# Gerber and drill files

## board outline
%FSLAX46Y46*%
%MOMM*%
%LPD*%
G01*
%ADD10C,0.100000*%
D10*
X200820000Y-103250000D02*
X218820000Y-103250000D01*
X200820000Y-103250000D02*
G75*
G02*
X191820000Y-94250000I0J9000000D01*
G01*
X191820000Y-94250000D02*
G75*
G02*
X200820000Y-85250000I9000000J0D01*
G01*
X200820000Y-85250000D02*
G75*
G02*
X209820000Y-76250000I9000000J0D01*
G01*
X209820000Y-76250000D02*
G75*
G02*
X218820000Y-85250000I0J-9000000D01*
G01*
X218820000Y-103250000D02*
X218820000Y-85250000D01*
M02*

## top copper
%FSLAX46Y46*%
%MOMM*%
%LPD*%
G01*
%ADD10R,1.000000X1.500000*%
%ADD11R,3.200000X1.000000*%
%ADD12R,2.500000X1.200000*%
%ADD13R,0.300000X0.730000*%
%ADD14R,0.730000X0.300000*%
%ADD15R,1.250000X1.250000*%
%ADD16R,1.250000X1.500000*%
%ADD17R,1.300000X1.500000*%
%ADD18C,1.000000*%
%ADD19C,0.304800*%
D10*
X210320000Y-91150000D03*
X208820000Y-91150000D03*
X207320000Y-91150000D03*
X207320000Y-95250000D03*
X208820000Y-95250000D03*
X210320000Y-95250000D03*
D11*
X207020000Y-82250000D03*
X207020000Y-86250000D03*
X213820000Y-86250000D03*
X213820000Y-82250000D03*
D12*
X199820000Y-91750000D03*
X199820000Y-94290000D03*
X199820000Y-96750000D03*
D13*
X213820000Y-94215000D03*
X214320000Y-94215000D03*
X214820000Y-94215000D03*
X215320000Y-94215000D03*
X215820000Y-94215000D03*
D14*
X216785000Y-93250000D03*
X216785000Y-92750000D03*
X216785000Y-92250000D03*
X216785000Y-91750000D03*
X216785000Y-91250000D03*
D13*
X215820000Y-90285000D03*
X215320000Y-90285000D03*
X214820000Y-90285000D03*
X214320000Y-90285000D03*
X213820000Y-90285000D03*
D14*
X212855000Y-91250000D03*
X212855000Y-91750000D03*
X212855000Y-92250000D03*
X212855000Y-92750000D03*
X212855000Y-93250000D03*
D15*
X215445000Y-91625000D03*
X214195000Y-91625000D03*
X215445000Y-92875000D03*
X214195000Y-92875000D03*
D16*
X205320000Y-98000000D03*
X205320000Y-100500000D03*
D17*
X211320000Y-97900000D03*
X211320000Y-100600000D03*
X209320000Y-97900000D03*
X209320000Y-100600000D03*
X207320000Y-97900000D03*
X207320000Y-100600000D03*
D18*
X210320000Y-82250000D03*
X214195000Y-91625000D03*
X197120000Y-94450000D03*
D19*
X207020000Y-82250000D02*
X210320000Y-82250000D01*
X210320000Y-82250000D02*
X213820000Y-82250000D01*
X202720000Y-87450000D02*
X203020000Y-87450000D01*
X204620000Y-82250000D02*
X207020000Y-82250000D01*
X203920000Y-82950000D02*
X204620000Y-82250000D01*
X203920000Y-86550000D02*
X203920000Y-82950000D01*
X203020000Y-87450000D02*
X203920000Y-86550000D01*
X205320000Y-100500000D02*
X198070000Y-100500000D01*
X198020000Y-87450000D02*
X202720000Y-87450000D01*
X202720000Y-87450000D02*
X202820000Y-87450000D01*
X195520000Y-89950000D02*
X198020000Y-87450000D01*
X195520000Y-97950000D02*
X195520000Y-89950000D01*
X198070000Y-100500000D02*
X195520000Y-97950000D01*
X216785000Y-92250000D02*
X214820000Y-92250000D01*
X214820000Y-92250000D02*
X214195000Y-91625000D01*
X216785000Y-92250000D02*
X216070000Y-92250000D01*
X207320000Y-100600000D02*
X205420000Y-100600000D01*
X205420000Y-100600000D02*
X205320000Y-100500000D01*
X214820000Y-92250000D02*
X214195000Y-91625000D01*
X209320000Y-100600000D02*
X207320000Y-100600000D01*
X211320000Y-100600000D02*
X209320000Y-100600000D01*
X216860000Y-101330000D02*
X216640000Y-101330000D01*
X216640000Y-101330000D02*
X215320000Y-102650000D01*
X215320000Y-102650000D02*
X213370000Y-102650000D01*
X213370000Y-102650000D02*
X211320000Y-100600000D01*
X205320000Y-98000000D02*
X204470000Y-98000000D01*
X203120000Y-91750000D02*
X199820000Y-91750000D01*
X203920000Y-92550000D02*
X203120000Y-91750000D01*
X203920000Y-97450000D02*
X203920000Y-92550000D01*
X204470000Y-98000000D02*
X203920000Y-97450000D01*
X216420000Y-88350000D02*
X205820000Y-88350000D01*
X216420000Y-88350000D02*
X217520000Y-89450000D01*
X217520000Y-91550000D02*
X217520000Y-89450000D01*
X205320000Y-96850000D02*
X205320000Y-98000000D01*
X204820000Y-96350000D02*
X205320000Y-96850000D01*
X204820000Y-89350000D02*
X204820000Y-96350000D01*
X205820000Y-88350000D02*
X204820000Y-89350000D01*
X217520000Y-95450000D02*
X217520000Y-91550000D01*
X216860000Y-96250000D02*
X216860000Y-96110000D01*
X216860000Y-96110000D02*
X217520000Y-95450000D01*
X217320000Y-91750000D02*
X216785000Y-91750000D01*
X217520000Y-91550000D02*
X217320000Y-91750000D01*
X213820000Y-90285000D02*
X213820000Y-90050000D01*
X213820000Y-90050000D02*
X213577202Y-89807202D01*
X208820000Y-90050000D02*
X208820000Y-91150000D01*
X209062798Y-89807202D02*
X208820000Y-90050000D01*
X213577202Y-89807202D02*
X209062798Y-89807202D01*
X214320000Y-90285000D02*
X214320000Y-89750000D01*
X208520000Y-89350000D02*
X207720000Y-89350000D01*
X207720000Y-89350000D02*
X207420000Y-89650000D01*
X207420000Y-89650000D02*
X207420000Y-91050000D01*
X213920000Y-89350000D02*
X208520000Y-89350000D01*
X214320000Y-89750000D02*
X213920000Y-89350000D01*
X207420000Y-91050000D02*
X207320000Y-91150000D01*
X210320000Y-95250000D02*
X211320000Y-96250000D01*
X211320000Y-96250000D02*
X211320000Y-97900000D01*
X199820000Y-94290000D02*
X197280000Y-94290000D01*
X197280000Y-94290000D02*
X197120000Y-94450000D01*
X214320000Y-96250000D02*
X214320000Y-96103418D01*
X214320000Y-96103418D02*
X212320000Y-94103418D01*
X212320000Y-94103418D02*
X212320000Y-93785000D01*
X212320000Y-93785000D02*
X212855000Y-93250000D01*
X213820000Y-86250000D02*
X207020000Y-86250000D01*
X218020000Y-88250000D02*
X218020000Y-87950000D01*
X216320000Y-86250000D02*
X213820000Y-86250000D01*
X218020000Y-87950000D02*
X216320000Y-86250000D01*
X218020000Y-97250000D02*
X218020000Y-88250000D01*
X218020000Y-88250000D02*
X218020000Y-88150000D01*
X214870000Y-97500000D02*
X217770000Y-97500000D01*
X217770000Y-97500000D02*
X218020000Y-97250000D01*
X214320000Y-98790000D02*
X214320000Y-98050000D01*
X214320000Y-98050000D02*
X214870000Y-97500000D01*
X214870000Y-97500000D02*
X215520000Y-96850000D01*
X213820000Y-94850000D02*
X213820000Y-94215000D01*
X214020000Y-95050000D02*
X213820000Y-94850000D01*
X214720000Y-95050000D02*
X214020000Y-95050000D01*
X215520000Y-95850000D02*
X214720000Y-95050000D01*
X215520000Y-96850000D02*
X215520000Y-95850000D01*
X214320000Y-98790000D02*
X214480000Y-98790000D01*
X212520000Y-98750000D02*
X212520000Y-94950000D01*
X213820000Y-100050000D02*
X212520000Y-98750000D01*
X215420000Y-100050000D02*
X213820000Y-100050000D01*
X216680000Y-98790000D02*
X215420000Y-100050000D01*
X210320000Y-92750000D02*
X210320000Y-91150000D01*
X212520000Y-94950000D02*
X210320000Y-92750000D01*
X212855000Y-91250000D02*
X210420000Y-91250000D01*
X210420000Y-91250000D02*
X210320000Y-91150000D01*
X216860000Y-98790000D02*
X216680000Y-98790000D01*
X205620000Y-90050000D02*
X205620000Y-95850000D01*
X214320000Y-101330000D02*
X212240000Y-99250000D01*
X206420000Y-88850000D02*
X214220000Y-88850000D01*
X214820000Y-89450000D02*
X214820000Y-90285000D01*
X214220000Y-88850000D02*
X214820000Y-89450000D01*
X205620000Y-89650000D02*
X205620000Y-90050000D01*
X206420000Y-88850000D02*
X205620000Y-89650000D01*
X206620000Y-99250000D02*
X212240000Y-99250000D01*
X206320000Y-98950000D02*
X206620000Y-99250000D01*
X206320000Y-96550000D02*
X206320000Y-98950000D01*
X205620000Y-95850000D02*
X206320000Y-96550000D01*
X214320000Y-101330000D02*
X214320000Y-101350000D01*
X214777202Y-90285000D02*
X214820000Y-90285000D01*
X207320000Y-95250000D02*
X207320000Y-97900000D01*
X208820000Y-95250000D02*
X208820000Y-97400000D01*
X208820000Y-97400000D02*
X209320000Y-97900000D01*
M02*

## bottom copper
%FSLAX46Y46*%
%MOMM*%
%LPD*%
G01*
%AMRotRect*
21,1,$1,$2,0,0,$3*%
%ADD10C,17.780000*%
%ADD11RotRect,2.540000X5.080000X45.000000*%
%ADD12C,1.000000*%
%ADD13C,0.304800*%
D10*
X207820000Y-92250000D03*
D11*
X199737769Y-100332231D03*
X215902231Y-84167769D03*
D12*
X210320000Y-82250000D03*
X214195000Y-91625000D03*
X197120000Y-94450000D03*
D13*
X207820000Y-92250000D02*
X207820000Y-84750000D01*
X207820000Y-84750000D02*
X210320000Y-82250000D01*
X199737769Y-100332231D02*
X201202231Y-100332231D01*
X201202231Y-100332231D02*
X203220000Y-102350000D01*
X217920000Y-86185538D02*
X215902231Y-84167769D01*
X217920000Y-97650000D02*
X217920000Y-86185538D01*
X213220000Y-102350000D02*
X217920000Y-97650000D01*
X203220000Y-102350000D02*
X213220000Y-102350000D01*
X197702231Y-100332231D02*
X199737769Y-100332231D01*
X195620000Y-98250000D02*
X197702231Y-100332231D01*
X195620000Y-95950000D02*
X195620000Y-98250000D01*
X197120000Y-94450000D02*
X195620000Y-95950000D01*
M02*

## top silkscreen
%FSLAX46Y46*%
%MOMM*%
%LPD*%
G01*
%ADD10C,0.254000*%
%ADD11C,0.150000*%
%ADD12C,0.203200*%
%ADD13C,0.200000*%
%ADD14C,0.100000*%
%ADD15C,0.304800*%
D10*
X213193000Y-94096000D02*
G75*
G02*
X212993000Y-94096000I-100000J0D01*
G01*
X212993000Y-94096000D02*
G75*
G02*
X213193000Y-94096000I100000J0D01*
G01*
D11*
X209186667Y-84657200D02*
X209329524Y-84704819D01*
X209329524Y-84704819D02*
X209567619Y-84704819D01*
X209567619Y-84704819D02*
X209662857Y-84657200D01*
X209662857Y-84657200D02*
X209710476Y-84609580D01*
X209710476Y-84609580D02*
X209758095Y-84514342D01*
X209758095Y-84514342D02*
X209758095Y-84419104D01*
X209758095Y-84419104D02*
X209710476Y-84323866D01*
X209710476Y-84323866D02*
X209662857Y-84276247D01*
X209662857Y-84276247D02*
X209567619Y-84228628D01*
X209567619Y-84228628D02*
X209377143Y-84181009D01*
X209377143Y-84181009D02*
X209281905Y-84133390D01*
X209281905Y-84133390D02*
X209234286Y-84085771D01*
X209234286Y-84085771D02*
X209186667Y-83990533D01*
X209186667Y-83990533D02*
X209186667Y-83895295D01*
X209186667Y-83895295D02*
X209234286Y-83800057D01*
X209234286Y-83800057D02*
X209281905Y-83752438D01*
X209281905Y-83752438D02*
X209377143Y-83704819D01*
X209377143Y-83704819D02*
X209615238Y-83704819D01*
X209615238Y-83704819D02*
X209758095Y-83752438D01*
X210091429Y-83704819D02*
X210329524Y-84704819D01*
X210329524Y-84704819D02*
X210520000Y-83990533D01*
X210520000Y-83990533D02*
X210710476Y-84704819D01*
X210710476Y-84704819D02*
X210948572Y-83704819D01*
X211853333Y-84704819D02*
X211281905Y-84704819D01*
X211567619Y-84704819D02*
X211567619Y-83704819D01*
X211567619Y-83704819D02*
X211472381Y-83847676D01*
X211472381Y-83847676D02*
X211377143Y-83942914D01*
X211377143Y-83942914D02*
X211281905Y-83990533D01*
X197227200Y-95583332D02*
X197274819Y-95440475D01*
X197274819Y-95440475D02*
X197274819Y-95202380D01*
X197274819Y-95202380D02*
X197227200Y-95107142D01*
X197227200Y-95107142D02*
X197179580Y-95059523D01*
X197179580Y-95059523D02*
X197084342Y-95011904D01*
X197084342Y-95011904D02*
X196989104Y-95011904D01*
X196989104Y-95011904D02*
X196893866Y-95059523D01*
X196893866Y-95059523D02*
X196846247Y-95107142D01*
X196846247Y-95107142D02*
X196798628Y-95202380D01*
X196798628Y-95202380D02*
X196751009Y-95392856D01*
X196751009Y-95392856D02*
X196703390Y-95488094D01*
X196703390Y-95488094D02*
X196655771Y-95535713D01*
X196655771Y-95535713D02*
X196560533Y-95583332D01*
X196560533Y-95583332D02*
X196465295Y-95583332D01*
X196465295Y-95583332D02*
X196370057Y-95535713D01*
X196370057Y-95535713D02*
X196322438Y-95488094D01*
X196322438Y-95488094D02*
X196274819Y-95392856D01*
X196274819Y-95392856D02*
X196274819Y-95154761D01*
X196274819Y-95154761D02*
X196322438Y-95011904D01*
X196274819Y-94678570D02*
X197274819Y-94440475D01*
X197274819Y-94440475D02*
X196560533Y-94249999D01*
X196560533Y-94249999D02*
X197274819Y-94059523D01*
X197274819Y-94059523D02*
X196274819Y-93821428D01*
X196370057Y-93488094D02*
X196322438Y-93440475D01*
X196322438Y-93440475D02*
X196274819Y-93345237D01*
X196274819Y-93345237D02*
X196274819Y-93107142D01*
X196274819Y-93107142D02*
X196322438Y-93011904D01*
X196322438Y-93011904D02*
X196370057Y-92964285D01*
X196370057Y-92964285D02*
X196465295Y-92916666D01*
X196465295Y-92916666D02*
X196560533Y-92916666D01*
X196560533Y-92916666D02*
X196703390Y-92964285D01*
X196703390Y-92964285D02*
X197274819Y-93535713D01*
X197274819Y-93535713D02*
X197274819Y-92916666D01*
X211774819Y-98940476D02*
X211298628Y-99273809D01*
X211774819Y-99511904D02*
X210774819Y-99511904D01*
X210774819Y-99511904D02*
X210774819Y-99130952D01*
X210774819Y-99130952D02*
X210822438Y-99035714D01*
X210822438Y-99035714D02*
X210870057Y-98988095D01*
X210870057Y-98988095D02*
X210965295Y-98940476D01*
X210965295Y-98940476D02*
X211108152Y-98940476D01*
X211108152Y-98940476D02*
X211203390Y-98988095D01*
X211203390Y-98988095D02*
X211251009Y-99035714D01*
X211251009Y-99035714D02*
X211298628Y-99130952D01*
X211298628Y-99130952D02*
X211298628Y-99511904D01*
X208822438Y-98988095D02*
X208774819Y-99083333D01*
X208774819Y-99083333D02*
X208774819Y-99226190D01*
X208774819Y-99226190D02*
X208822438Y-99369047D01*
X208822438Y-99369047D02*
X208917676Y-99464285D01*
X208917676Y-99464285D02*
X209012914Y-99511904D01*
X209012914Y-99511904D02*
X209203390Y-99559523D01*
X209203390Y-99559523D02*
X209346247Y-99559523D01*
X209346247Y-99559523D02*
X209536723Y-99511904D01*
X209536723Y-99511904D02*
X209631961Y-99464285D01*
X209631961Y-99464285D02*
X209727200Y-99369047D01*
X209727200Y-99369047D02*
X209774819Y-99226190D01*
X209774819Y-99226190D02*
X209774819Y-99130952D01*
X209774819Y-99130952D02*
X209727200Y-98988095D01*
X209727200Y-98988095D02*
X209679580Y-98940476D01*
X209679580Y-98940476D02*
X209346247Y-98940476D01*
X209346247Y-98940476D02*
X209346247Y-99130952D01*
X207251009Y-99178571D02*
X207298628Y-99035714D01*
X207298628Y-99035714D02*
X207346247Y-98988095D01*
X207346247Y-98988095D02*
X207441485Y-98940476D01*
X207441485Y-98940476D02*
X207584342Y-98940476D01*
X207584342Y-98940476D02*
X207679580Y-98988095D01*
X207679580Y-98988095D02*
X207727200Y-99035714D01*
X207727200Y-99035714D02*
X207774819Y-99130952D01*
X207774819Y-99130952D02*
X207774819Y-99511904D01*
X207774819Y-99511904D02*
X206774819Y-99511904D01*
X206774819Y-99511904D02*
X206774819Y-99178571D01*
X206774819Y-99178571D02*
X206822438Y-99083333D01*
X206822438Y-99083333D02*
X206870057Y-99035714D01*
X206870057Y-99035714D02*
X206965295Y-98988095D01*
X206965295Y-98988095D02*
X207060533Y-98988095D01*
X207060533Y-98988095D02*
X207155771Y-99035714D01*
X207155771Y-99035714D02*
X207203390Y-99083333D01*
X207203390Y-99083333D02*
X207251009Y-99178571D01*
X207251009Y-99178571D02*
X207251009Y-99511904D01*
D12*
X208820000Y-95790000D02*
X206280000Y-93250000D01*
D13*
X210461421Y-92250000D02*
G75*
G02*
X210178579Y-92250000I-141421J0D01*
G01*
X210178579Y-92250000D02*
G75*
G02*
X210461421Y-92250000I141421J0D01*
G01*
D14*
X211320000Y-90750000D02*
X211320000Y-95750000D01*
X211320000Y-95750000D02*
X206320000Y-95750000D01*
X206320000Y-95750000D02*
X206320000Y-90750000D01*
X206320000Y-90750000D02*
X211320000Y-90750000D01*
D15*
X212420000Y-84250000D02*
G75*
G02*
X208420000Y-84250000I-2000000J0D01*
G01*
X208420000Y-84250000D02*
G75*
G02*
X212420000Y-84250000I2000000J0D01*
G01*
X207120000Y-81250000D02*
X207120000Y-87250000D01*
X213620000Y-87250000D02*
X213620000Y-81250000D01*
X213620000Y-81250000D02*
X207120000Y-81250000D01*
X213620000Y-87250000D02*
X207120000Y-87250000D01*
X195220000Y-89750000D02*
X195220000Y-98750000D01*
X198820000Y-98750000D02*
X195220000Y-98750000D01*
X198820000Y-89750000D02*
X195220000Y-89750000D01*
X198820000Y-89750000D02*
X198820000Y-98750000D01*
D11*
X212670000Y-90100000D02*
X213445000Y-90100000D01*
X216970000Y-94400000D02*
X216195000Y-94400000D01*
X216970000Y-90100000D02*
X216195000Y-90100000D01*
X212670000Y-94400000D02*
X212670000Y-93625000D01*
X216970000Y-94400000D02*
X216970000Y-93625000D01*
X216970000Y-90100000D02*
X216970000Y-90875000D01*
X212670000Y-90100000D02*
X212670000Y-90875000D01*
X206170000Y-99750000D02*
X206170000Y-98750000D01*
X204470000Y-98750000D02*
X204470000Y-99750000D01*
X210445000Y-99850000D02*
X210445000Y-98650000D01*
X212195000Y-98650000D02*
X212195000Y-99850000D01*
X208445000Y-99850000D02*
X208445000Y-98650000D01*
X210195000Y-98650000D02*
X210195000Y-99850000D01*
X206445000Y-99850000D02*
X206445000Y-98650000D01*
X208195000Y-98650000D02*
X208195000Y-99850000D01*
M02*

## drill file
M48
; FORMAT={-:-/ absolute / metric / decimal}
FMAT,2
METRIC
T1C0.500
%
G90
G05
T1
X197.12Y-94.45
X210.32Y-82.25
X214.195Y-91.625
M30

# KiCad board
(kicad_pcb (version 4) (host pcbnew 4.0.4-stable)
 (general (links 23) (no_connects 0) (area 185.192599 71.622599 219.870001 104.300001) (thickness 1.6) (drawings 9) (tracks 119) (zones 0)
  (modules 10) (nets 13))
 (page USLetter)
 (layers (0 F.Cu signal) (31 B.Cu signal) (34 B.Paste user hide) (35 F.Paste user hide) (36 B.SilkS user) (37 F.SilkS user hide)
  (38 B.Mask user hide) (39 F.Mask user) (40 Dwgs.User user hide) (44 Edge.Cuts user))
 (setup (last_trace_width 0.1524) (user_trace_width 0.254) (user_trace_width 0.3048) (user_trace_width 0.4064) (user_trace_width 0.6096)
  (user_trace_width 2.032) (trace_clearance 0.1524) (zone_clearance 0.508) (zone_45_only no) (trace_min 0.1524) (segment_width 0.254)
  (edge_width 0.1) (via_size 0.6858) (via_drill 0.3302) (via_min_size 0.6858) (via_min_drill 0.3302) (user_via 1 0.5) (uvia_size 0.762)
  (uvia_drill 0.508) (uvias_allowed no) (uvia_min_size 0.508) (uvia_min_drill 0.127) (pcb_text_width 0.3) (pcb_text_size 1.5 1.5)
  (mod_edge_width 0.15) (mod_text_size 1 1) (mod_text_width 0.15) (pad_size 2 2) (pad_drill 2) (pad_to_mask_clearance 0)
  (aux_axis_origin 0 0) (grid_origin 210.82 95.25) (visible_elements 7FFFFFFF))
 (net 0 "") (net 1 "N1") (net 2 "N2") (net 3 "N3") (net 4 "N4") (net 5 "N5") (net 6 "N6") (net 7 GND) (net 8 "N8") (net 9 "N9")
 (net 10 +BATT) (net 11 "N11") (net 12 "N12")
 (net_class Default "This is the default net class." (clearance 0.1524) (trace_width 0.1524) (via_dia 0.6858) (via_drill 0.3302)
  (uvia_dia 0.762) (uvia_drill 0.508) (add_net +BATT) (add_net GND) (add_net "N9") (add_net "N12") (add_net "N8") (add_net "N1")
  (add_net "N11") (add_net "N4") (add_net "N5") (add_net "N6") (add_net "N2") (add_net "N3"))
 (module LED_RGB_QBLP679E (layer F.Cu) (at 208.82 93.25 270)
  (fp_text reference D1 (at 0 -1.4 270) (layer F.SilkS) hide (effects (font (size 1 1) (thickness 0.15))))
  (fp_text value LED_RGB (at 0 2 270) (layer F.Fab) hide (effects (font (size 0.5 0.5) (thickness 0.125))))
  (fp_line (start 2.54 0) (end 0 2.54) (layer F.SilkS) (width 0.2032))
  (fp_circle (center -1 -1.5) (end -1.1 -1.6) (layer F.SilkS) (width 0.2))
  (fp_line (start -2.5 -2.5) (end 2.5 -2.5) (layer F.SilkS) (width 0.1))
  (fp_line (start 2.5 -2.5) (end 2.5 2.5) (layer F.SilkS) (width 0.1))
  (fp_line (start 2.5 2.5) (end -2.5 2.5) (layer F.SilkS) (width 0.1))
  (fp_line (start -2.5 2.5) (end -2.5 -2.5) (layer F.SilkS) (width 0.1))
  (pad 4 smd rect (at -2.1 -1.5) (size 1 1.5) (layers F.Cu F.Paste F.Mask) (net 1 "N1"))
  (pad 5 smd rect (at -2.1 0) (size 1 1.5) (layers F.Cu F.Paste F.Mask) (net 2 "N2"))
  (pad 6 smd rect (at -2.1 1.5) (size 1 1.5) (layers F.Cu F.Paste F.Mask) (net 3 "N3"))
  (pad 1 smd rect (at 2 1.5) (size 1 1.5) (layers F.Cu F.Paste F.Mask) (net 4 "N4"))
  (pad 2 smd rect (at 2 0) (size 1 1.5) (layers F.Cu F.Paste F.Mask) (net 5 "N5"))
  (pad 3 smd rect (at 2 -1.5) (size 1 1.5) (layers F.Cu F.Paste F.Mask) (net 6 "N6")))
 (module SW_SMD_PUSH (layer F.Cu) (at 213.82 86.25 180)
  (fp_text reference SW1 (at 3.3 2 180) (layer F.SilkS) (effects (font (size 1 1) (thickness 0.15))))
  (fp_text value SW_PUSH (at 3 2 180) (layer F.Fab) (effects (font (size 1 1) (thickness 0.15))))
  (fp_circle (center 3.4 2) (end 3.4 0) (layer F.SilkS) (width 0.3048))
  (fp_line (start 6.7 5) (end 6.7 -1) (layer F.SilkS) (width 0.3048))
  (fp_line (start 0.2 -1) (end 0.2 5) (layer F.SilkS) (width 0.3048))
  (fp_line (start 0.2 5) (end 6.7 5) (layer F.SilkS) (width 0.3048))
  (fp_line (start 0.2 -1) (end 6.7 -1) (layer F.SilkS) (width 0.3048))
  (pad 2 smd rect (at 6.8 4 180) (size 3.2 1) (layers F.Cu F.Paste F.Mask) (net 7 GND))
  (pad 1 smd rect (at 6.8 0 180) (size 3.2 1) (layers F.Cu F.Paste F.Mask) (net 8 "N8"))
  (pad 1 smd rect (at 0 0 180) (size 3.2 1) (layers F.Cu F.Paste F.Mask) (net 8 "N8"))
  (pad 2 smd rect (at 0 4 180) (size 3.2 1) (layers F.Cu F.Paste F.Mask) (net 7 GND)))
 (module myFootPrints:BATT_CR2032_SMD (layer B.Cu) (at 207.82 92.25 45)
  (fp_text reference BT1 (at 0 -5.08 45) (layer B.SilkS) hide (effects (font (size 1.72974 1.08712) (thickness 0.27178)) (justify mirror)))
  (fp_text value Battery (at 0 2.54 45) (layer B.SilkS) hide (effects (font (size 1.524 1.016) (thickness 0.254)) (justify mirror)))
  (pad 2 smd circle (at 0 0 45) (size 17.78 17.78) (layers B.Cu B.Paste B.Mask) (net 7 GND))
  (pad 1 smd rect (at -11.43 0 45) (size 2.54 5.08) (layers B.Cu B.Paste B.Mask) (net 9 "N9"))
  (pad 1 smd rect (at 11.43 0 45) (size 2.54 5.08) (layers B.Cu B.Paste B.Mask) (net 9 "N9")))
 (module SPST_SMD (layer F.Cu) (at 199.82 94.25 270)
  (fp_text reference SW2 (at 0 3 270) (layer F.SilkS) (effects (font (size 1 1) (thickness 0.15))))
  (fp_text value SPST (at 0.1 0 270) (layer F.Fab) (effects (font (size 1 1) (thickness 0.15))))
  (fp_line (start -4.5 4.6) (end 4.5 4.6) (layer F.SilkS) (width 0.3048))
  (fp_line (start 4.5 1) (end 4.5 4.6) (layer F.SilkS) (width 0.3048))
  (fp_line (start -4.5 1) (end -4.5 4.6) (layer F.SilkS) (width 0.3048))
  (fp_line (start -4.5 1) (end 4.5 1) (layer F.SilkS) (width 0.3048))
  (pad 1 smd rect (at -2.5 0 270) (size 1.2 2.5) (layers F.Cu F.Paste F.Mask) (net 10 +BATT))
  (pad 2 smd rect (at 0.04 0 270) (size 1.2 2.5) (layers F.Cu F.Paste F.Mask) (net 9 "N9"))
  (pad 3 smd rect (at 2.5 0 270) (size 1.2 2.5) (layers F.Cu F.Paste F.Mask)))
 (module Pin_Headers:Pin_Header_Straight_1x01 (layer F.Cu) (at 208.32 78.25)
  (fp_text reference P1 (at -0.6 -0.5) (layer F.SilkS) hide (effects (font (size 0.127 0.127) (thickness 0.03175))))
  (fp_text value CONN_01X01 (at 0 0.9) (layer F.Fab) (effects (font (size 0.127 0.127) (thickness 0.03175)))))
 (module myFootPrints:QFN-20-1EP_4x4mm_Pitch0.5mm (layer F.Cu) (at 214.82 92.25 90)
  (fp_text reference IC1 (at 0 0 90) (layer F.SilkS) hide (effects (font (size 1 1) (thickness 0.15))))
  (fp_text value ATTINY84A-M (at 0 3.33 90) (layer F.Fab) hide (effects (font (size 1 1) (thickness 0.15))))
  (fp_line (start 2.15 -2.15) (end 2.15 -1.375) (layer F.SilkS) (width 0.15))
  (fp_line (start -2.15 2.15) (end -2.15 1.375) (layer F.SilkS) (width 0.15))
  (fp_line (start 2.15 2.15) (end 2.15 1.375) (layer F.SilkS) (width 0.15))
  (fp_line (start -2.15 -2.15) (end -1.375 -2.15) (layer F.SilkS) (width 0.15))
  (fp_line (start -2.15 2.15) (end -1.375 2.15) (layer F.SilkS) (width 0.15))
  (fp_line (start 2.15 2.15) (end 1.375 2.15) (layer F.SilkS) (width 0.15))
  (fp_line (start 2.15 -2.15) (end 1.375 -2.15) (layer F.SilkS) (width 0.15))
  (pad 1 smd rect (at -1.965 -1 90) (size 0.73 0.3) (layers F.Cu F.Paste F.Mask) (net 8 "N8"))
  (pad 2 smd rect (at -1.965 -0.5 90) (size 0.73 0.3) (layers F.Cu F.Paste F.Mask))
  (pad 3 smd rect (at -1.965 0 90) (size 0.73 0.3) (layers F.Cu F.Paste F.Mask))
  (pad 4 smd rect (at -1.965 0.5 90) (size 0.73 0.3) (layers F.Cu F.Paste F.Mask))
  (pad 5 smd rect (at -1.965 1 90) (size 0.73 0.3) (layers F.Cu F.Paste F.Mask))
  (pad 6 smd rect (at -1 1.965 180) (size 0.73 0.3) (layers F.Cu F.Paste F.Mask))
  (pad 7 smd rect (at -0.5 1.965 180) (size 0.73 0.3) (layers F.Cu F.Paste F.Mask))
  (pad 8 smd rect (at 0 1.965 180) (size 0.73 0.3) (layers F.Cu F.Paste F.Mask) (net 7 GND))
  (pad 9 smd rect (at 0.5 1.965 180) (size 0.73 0.3) (layers F.Cu F.Paste F.Mask) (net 10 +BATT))
  (pad 10 smd rect (at 1 1.965 180) (size 0.73 0.3) (layers F.Cu F.Paste F.Mask))
  (pad 11 smd rect (at 1.965 1 90) (size 0.73 0.3) (layers F.Cu F.Paste F.Mask))
  (pad 12 smd rect (at 1.965 0.5 90) (size 0.73 0.3) (layers F.Cu F.Paste F.Mask))
  (pad 13 smd rect (at 1.965 0 90) (size 0.73 0.3) (layers F.Cu F.Paste F.Mask) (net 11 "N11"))
  (pad 14 smd rect (at 1.965 -0.5 90) (size 0.73 0.3) (layers F.Cu F.Paste F.Mask) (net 3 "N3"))
  (pad 15 smd rect (at 1.965 -1 90) (size 0.73 0.3) (layers F.Cu F.Paste F.Mask) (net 2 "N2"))
  (pad 16 smd rect (at 1 -1.965 180) (size 0.73 0.3) (layers F.Cu F.Paste F.Mask) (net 1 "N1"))
  (pad 17 smd rect (at 0.5 -1.965 180) (size 0.73 0.3) (layers F.Cu F.Paste F.Mask))
  (pad 18 smd rect (at 0 -1.965 180) (size 0.73 0.3) (layers F.Cu F.Paste F.Mask))
  (pad 19 smd rect (at -0.5 -1.965 180) (size 0.73 0.3) (layers F.Cu F.Paste F.Mask))
  (pad 20 smd rect (at -1 -1.965 180) (size 0.73 0.3) (layers F.Cu F.Paste F.Mask) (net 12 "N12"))
  (pad 8 smd rect (at 0.625 0.625 90) (size 1.25 1.25) (layers F.Cu F.Paste F.Mask) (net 7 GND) (solder_paste_margin_ratio -0.2))
  (pad 8 smd rect (at 0.625 -0.625 90) (size 1.25 1.25) (layers F.Cu F.Paste F.Mask) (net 7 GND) (solder_paste_margin_ratio -0.2))
  (pad 8 smd rect (at -0.625 0.625 90) (size 1.25 1.25) (layers F.Cu F.Paste F.Mask) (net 7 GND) (solder_paste_margin_ratio -0.2))
  (pad 8 smd rect (at -0.625 -0.625 90) (size 1.25 1.25) (layers F.Cu F.Paste F.Mask) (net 7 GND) (solder_paste_margin_ratio -0.2)))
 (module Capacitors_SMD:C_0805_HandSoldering (layer F.Cu) (at 205.32 99.25 270)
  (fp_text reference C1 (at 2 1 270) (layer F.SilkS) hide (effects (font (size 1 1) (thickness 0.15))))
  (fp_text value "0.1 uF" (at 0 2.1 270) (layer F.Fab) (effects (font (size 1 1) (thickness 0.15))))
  (fp_line (start 0.5 -0.85) (end -0.5 -0.85) (layer F.SilkS) (width 0.15))
  (fp_line (start -0.5 0.85) (end 0.5 0.85) (layer F.SilkS) (width 0.15))
  (pad 1 smd rect (at -1.25 0 270) (size 1.5 1.25) (layers F.Cu F.Paste F.Mask) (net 10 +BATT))
  (pad 2 smd rect (at 1.25 0 270) (size 1.5 1.25) (layers F.Cu F.Paste F.Mask) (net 7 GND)))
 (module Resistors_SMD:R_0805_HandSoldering (layer F.Cu) (at 211.32 99.25 270)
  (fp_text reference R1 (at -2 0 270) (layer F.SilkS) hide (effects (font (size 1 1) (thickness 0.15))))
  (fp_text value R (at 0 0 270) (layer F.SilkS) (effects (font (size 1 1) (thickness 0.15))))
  (fp_line (start 0.6 0.875) (end -0.6 0.875) (layer F.SilkS) (width 0.15))
  (fp_line (start -0.6 -0.875) (end 0.6 -0.875) (layer F.SilkS) (width 0.15))
  (pad 1 smd rect (at -1.35 0 270) (size 1.5 1.3) (layers F.Cu F.Paste F.Mask) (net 6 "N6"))
  (pad 2 smd rect (at 1.35 0 270) (size 1.5 1.3) (layers F.Cu F.Paste F.Mask) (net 7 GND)))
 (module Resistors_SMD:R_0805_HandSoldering (layer F.Cu) (at 209.32 99.25 270)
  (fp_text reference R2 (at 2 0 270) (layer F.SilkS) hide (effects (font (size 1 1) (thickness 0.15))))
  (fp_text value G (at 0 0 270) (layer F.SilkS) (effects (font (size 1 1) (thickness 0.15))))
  (fp_line (start 0.6 0.875) (end -0.6 0.875) (layer F.SilkS) (width 0.15))
  (fp_line (start -0.6 -0.875) (end 0.6 -0.875) (layer F.SilkS) (width 0.15))
  (pad 1 smd rect (at -1.35 0 270) (size 1.5 1.3) (layers F.Cu F.Paste F.Mask) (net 5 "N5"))
  (pad 2 smd rect (at 1.35 0 270) (size 1.5 1.3) (layers F.Cu F.Paste F.Mask) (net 7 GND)))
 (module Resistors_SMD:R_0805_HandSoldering (layer F.Cu) (at 207.32 99.25 270)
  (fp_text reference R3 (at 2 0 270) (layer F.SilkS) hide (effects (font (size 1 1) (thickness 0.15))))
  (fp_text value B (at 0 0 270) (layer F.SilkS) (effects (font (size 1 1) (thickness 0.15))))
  (fp_line (start 0.6 0.875) (end -0.6 0.875) (layer F.SilkS) (width 0.15))
  (fp_line (start -0.6 -0.875) (end 0.6 -0.875) (layer F.SilkS) (width 0.15))
  (pad 1 smd rect (at -1.35 0 270) (size 1.5 1.3) (layers F.Cu F.Paste F.Mask) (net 4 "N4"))
  (pad 2 smd rect (at 1.35 0 270) (size 1.5 1.3) (layers F.Cu F.Paste F.Mask) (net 7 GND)))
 (gr_circle (center 213.093 94.096) (end 213.193 94.096) (layer F.SilkS) (width 0.254))
 (gr_line (start 200.82 103.25) (end 218.82 103.25) (angle 90) (layer Edge.Cuts) (width 0.1))
 (gr_arc (start 200.82 94.25) (end 200.82 103.25) (angle 90) (layer Edge.Cuts) (width 0.1))
 (gr_arc (start 200.82 94.25) (end 191.82 94.25) (angle 90) (layer Edge.Cuts) (width 0.1))
 (gr_arc (start 209.82 85.25) (end 200.82 85.25) (angle 90) (layer Edge.Cuts) (width 0.1))
 (gr_arc (start 209.82 85.25) (end 209.82 76.25) (angle 90) (layer Edge.Cuts) (width 0.1))
 (gr_line (start 218.82 103.25) (end 218.82 85.25) (angle 90) (layer Edge.Cuts) (width 0.1))
 (segment (start 207.02 82.25) (end 210.32 82.25) (width 0.3048) (layer F.Cu) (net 7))
 (segment (start 207.82 92.25) (end 207.82 84.75) (width 0.3048) (layer B.Cu) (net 7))
 (segment (start 207.82 84.75) (end 210.32 82.25) (width 0.3048) (layer B.Cu) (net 7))
 (via (at 210.32 82.25) (size 1) (drill 0.5) (layers F.Cu B.Cu) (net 7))
 (segment (start 210.32 82.25) (end 213.82 82.25) (width 0.3048) (layer F.Cu) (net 7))
 (segment (start 202.72 87.45) (end 203.02 87.45) (width 0.3048) (layer F.Cu) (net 7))
 (segment (start 204.62 82.25) (end 207.02 82.25) (width 0.3048) (layer F.Cu) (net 7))
 (segment (start 203.92 82.95) (end 204.62 82.25) (width 0.3048) (layer F.Cu) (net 7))
 (segment (start 203.92 86.55) (end 203.92 82.95) (width 0.3048) (layer F.Cu) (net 7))
 (segment (start 203.02 87.45) (end 203.92 86.55) (width 0.3048) (layer F.Cu) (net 7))
 (segment (start 205.32 100.5) (end 198.07 100.5) (width 0.3048) (layer F.Cu) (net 7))
 (segment (start 198.02 87.45) (end 202.72 87.45) (width 0.3048) (layer F.Cu) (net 7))
 (segment (start 202.72 87.45) (end 202.82 87.45) (width 0.3048) (layer F.Cu) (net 7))
 (segment (start 195.52 89.95) (end 198.02 87.45) (width 0.3048) (layer F.Cu) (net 7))
 (segment (start 195.52 97.95) (end 195.52 89.95) (width 0.3048) (layer F.Cu) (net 7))
 (segment (start 198.07 100.5) (end 195.52 97.95) (width 0.3048) (layer F.Cu) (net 7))
 (segment (start 216.785 92.25) (end 214.82 92.25) (width 0.3048) (layer F.Cu) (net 7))
 (segment (start 214.82 92.25) (end 214.195 91.625) (width 0.3048) (layer F.Cu) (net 7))
 (via (at 214.195 91.625) (size 1) (drill 0.5) (layers F.Cu B.Cu) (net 7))
 (segment (start 216.785 92.25) (end 216.07 92.25) (width 0.3048) (layer F.Cu) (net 7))
 (segment (start 207.32 100.6) (end 205.42 100.6) (width 0.3048) (layer F.Cu) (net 7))
 (segment (start 205.42 100.6) (end 205.32 100.5) (width 0.3048) (layer F.Cu) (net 7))
 (segment (start 214.82 92.25) (end 214.195 91.625) (width 0.3048) (layer F.Cu) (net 7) (status 30))
 (segment (start 209.32 100.6) (end 207.32 100.6) (width 0.3048) (layer F.Cu) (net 7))
 (segment (start 211.32 100.6) (end 209.32 100.6) (width 0.3048) (layer F.Cu) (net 7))
 (segment (start 216.86 101.33) (end 216.64 101.33) (width 0.3048) (layer F.Cu) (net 7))
 (segment (start 216.64 101.33) (end 215.32 102.65) (width 0.3048) (layer F.Cu) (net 7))
 (segment (start 215.32 102.65) (end 213.37 102.65) (width 0.3048) (layer F.Cu) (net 7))
 (segment (start 213.37 102.65) (end 211.32 100.6) (width 0.3048) (layer F.Cu) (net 7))
 (segment (start 205.32 98) (end 204.47 98) (width 0.3048) (layer F.Cu) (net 10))
 (segment (start 203.12 91.75) (end 199.82 91.75) (width 0.3048) (layer F.Cu) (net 10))
 (segment (start 203.92 92.55) (end 203.12 91.75) (width 0.3048) (layer F.Cu) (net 10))
 (segment (start 203.92 97.45) (end 203.92 92.55) (width 0.3048) (layer F.Cu) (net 10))
 (segment (start 204.47 98) (end 203.92 97.45) (width 0.3048) (layer F.Cu) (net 10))
 (segment (start 216.42 88.35) (end 205.82 88.35) (width 0.3048) (layer F.Cu) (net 10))
 (segment (start 216.42 88.35) (end 217.52 89.45) (width 0.3048) (layer F.Cu) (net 10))
 (segment (start 217.52 91.55) (end 217.52 89.45) (width 0.3048) (layer F.Cu) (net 10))
 (segment (start 205.32 96.85) (end 205.32 98) (width 0.3048) (layer F.Cu) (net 10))
 (segment (start 204.82 96.35) (end 205.32 96.85) (width 0.3048) (layer F.Cu) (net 10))
 (segment (start 204.82 89.35) (end 204.82 96.35) (width 0.3048) (layer F.Cu) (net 10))
 (segment (start 205.82 88.35) (end 204.82 89.35) (width 0.3048) (layer F.Cu) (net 10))
 (segment (start 217.52 95.45) (end 217.52 91.55) (width 0.3048) (layer F.Cu) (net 10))
 (segment (start 216.86 96.25) (end 216.86 96.11) (width 0.3048) (layer F.Cu) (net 10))
 (segment (start 216.86 96.11) (end 217.52 95.45) (width 0.3048) (layer F.Cu) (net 10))
 (segment (start 217.32 91.75) (end 216.785 91.75) (width 0.3048) (layer F.Cu) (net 10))
 (segment (start 217.52 91.55) (end 217.32 91.75) (width 0.3048) (layer F.Cu) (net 10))
 (segment (start 213.82 90.285) (end 213.82 90.05) (width 0.3048) (layer F.Cu) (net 2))
 (segment (start 213.82 90.05) (end 213.577202 89.807202) (width 0.3048) (layer F.Cu) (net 2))
 (segment (start 208.82 90.05) (end 208.82 91.15) (width 0.3048) (layer F.Cu) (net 2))
 (segment (start 209.062798 89.807202) (end 208.82 90.05) (width 0.3048) (layer F.Cu) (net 2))
 (segment (start 213.577202 89.807202) (end 209.062798 89.807202) (width 0.3048) (layer F.Cu) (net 2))
 (segment (start 214.32 90.285) (end 214.32 89.75) (width 0.3048) (layer F.Cu) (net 3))
 (segment (start 208.52 89.35) (end 207.72 89.35) (width 0.3048) (layer F.Cu) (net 3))
 (segment (start 207.72 89.35) (end 207.42 89.65) (width 0.3048) (layer F.Cu) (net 3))
 (segment (start 207.42 89.65) (end 207.42 91.05) (width 0.3048) (layer F.Cu) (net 3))
 (segment (start 213.92 89.35) (end 208.52 89.35) (width 0.3048) (layer F.Cu) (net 3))
 (segment (start 214.32 89.75) (end 213.92 89.35) (width 0.3048) (layer F.Cu) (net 3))
 (segment (start 207.42 91.05) (end 207.32 91.15) (width 0.3048) (layer F.Cu) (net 3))
 (segment (start 210.32 95.25) (end 211.32 96.25) (width 0.3048) (layer F.Cu) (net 6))
 (segment (start 211.32 96.25) (end 211.32 97.9) (width 0.3048) (layer F.Cu) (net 6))
 (segment (start 199.737769 100.332231) (end 201.202231 100.332231) (width 0.3048) (layer B.Cu) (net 9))
 (segment (start 201.202231 100.332231) (end 203.22 102.35) (width 0.3048) (layer B.Cu) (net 9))
 (segment (start 217.92 86.185538) (end 215.902231 84.167769) (width 0.3048) (layer B.Cu) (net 9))
 (segment (start 217.92 97.65) (end 217.92 86.185538) (width 0.3048) (layer B.Cu) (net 9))
 (segment (start 213.22 102.35) (end 217.92 97.65) (width 0.3048) (layer B.Cu) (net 9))
 (segment (start 203.22 102.35) (end 213.22 102.35) (width 0.3048) (layer B.Cu) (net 9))
 (segment (start 199.82 94.29) (end 197.28 94.29) (width 0.3048) (layer F.Cu) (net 9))
 (segment (start 197.702231 100.332231) (end 199.737769 100.332231) (width 0.3048) (layer B.Cu) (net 9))
 (segment (start 195.62 98.25) (end 197.702231 100.332231) (width 0.3048) (layer B.Cu) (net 9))
 (segment (start 195.62 95.95) (end 195.62 98.25) (width 0.3048) (layer B.Cu) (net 9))
 (segment (start 197.12 94.45) (end 195.62 95.95) (width 0.3048) (layer B.Cu) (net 9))
 (via (at 197.12 94.45) (size 1) (drill 0.5) (layers F.Cu B.Cu) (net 9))
 (segment (start 197.28 94.29) (end 197.12 94.45) (width 0.3048) (layer F.Cu) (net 9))
 (segment (start 214.32 96.25) (end 214.32 96.103418) (width 0.3048) (layer F.Cu) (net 12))
 (segment (start 214.32 96.103418) (end 212.32 94.103418) (width 0.3048) (layer F.Cu) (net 12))
 (segment (start 212.32 94.103418) (end 212.32 93.785) (width 0.3048) (layer F.Cu) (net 12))
 (segment (start 212.32 93.785) (end 212.855 93.25) (width 0.3048) (layer F.Cu) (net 12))
 (segment (start 213.82 86.25) (end 207.02 86.25) (width 0.3048) (layer F.Cu) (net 8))
 (segment (start 218.02 88.25) (end 218.02 87.95) (width 0.3048) (layer F.Cu) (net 8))
 (segment (start 216.32 86.25) (end 213.82 86.25) (width 0.3048) (layer F.Cu) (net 8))
 (segment (start 218.02 87.95) (end 216.32 86.25) (width 0.3048) (layer F.Cu) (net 8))
 (segment (start 218.02 97.25) (end 218.02 88.25) (width 0.3048) (layer F.Cu) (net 8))
 (segment (start 218.02 88.25) (end 218.02 88.15) (width 0.3048) (layer F.Cu) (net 8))
 (segment (start 214.87 97.5) (end 217.77 97.5) (width 0.3048) (layer F.Cu) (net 8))
 (segment (start 217.77 97.5) (end 218.02 97.25) (width 0.3048) (layer F.Cu) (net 8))
 (segment (start 214.32 98.79) (end 214.32 98.05) (width 0.3048) (layer F.Cu) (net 8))
 (segment (start 214.32 98.05) (end 214.87 97.5) (width 0.3048) (layer F.Cu) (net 8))
 (segment (start 214.87 97.5) (end 215.52 96.85) (width 0.3048) (layer F.Cu) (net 8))
 (segment (start 213.82 94.85) (end 213.82 94.215) (width 0.3048) (layer F.Cu) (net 8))
 (segment (start 214.02 95.05) (end 213.82 94.85) (width 0.3048) (layer F.Cu) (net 8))
 (segment (start 214.72 95.05) (end 214.02 95.05) (width 0.3048) (layer F.Cu) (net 8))
 (segment (start 215.52 95.85) (end 214.72 95.05) (width 0.3048) (layer F.Cu) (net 8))
 (segment (start 215.52 96.85) (end 215.52 95.85) (width 0.3048) (layer F.Cu) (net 8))
 (segment (start 214.32 98.79) (end 214.48 98.79) (width 0.3048) (layer F.Cu) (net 8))
 (segment (start 212.52 98.75) (end 212.52 94.95) (width 0.3048) (layer F.Cu) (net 1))
 (segment (start 213.82 100.05) (end 212.52 98.75) (width 0.3048) (layer F.Cu) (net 1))
 (segment (start 215.42 100.05) (end 213.82 100.05) (width 0.3048) (layer F.Cu) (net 1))
 (segment (start 216.68 98.79) (end 215.42 100.05) (width 0.3048) (layer F.Cu) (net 1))
 (segment (start 210.32 92.75) (end 210.32 91.15) (width 0.3048) (layer F.Cu) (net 1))
 (segment (start 212.52 94.95) (end 210.32 92.75) (width 0.3048) (layer F.Cu) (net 1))
 (segment (start 212.855 91.25) (end 210.42 91.25) (width 0.3048) (layer F.Cu) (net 1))
 (segment (start 210.42 91.25) (end 210.32 91.15) (width 0.3048) (layer F.Cu) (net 1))
 (segment (start 216.86 98.79) (end 216.68 98.79) (width 0.3048) (layer F.Cu) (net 1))
 (segment (start 205.62 90.05) (end 205.62 95.85) (width 0.3048) (layer F.Cu) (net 11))
 (segment (start 214.32 101.33) (end 212.24 99.25) (width 0.3048) (layer F.Cu) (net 11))
 (segment (start 206.42 88.85) (end 214.22 88.85) (width 0.3048) (layer F.Cu) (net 11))
 (segment (start 214.82 89.45) (end 214.82 90.285) (width 0.3048) (layer F.Cu) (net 11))
 (segment (start 214.22 88.85) (end 214.82 89.45) (width 0.3048) (layer F.Cu) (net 11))
 (segment (start 205.62 89.65) (end 205.62 90.05) (width 0.3048) (layer F.Cu) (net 11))
 (segment (start 206.42 88.85) (end 205.62 89.65) (width 0.3048) (layer F.Cu) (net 11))
 (segment (start 206.62 99.25) (end 212.24 99.25) (width 0.3048) (layer F.Cu) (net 11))
 (segment (start 206.32 98.95) (end 206.62 99.25) (width 0.3048) (layer F.Cu) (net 11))
 (segment (start 206.32 96.55) (end 206.32 98.95) (width 0.3048) (layer F.Cu) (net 11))
 (segment (start 205.62 95.85) (end 206.32 96.55) (width 0.3048) (layer F.Cu) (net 11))
 (segment (start 214.32 101.33) (end 214.32 101.35) (width 0.3048) (layer F.Cu) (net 11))
 (segment (start 214.777202 90.285) (end 214.82 90.285) (width 0.3048) (layer F.Cu) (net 11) (status 30))
 (segment (start 207.32 95.25) (end 207.32 97.9) (width 0.3048) (layer F.Cu) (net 4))
 (segment (start 208.82 95.25) (end 208.82 97.4) (width 0.3048) (layer F.Cu) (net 5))
 (segment (start 208.82 97.4) (end 209.32 97.9) (width 0.3048) (layer F.Cu) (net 5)))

